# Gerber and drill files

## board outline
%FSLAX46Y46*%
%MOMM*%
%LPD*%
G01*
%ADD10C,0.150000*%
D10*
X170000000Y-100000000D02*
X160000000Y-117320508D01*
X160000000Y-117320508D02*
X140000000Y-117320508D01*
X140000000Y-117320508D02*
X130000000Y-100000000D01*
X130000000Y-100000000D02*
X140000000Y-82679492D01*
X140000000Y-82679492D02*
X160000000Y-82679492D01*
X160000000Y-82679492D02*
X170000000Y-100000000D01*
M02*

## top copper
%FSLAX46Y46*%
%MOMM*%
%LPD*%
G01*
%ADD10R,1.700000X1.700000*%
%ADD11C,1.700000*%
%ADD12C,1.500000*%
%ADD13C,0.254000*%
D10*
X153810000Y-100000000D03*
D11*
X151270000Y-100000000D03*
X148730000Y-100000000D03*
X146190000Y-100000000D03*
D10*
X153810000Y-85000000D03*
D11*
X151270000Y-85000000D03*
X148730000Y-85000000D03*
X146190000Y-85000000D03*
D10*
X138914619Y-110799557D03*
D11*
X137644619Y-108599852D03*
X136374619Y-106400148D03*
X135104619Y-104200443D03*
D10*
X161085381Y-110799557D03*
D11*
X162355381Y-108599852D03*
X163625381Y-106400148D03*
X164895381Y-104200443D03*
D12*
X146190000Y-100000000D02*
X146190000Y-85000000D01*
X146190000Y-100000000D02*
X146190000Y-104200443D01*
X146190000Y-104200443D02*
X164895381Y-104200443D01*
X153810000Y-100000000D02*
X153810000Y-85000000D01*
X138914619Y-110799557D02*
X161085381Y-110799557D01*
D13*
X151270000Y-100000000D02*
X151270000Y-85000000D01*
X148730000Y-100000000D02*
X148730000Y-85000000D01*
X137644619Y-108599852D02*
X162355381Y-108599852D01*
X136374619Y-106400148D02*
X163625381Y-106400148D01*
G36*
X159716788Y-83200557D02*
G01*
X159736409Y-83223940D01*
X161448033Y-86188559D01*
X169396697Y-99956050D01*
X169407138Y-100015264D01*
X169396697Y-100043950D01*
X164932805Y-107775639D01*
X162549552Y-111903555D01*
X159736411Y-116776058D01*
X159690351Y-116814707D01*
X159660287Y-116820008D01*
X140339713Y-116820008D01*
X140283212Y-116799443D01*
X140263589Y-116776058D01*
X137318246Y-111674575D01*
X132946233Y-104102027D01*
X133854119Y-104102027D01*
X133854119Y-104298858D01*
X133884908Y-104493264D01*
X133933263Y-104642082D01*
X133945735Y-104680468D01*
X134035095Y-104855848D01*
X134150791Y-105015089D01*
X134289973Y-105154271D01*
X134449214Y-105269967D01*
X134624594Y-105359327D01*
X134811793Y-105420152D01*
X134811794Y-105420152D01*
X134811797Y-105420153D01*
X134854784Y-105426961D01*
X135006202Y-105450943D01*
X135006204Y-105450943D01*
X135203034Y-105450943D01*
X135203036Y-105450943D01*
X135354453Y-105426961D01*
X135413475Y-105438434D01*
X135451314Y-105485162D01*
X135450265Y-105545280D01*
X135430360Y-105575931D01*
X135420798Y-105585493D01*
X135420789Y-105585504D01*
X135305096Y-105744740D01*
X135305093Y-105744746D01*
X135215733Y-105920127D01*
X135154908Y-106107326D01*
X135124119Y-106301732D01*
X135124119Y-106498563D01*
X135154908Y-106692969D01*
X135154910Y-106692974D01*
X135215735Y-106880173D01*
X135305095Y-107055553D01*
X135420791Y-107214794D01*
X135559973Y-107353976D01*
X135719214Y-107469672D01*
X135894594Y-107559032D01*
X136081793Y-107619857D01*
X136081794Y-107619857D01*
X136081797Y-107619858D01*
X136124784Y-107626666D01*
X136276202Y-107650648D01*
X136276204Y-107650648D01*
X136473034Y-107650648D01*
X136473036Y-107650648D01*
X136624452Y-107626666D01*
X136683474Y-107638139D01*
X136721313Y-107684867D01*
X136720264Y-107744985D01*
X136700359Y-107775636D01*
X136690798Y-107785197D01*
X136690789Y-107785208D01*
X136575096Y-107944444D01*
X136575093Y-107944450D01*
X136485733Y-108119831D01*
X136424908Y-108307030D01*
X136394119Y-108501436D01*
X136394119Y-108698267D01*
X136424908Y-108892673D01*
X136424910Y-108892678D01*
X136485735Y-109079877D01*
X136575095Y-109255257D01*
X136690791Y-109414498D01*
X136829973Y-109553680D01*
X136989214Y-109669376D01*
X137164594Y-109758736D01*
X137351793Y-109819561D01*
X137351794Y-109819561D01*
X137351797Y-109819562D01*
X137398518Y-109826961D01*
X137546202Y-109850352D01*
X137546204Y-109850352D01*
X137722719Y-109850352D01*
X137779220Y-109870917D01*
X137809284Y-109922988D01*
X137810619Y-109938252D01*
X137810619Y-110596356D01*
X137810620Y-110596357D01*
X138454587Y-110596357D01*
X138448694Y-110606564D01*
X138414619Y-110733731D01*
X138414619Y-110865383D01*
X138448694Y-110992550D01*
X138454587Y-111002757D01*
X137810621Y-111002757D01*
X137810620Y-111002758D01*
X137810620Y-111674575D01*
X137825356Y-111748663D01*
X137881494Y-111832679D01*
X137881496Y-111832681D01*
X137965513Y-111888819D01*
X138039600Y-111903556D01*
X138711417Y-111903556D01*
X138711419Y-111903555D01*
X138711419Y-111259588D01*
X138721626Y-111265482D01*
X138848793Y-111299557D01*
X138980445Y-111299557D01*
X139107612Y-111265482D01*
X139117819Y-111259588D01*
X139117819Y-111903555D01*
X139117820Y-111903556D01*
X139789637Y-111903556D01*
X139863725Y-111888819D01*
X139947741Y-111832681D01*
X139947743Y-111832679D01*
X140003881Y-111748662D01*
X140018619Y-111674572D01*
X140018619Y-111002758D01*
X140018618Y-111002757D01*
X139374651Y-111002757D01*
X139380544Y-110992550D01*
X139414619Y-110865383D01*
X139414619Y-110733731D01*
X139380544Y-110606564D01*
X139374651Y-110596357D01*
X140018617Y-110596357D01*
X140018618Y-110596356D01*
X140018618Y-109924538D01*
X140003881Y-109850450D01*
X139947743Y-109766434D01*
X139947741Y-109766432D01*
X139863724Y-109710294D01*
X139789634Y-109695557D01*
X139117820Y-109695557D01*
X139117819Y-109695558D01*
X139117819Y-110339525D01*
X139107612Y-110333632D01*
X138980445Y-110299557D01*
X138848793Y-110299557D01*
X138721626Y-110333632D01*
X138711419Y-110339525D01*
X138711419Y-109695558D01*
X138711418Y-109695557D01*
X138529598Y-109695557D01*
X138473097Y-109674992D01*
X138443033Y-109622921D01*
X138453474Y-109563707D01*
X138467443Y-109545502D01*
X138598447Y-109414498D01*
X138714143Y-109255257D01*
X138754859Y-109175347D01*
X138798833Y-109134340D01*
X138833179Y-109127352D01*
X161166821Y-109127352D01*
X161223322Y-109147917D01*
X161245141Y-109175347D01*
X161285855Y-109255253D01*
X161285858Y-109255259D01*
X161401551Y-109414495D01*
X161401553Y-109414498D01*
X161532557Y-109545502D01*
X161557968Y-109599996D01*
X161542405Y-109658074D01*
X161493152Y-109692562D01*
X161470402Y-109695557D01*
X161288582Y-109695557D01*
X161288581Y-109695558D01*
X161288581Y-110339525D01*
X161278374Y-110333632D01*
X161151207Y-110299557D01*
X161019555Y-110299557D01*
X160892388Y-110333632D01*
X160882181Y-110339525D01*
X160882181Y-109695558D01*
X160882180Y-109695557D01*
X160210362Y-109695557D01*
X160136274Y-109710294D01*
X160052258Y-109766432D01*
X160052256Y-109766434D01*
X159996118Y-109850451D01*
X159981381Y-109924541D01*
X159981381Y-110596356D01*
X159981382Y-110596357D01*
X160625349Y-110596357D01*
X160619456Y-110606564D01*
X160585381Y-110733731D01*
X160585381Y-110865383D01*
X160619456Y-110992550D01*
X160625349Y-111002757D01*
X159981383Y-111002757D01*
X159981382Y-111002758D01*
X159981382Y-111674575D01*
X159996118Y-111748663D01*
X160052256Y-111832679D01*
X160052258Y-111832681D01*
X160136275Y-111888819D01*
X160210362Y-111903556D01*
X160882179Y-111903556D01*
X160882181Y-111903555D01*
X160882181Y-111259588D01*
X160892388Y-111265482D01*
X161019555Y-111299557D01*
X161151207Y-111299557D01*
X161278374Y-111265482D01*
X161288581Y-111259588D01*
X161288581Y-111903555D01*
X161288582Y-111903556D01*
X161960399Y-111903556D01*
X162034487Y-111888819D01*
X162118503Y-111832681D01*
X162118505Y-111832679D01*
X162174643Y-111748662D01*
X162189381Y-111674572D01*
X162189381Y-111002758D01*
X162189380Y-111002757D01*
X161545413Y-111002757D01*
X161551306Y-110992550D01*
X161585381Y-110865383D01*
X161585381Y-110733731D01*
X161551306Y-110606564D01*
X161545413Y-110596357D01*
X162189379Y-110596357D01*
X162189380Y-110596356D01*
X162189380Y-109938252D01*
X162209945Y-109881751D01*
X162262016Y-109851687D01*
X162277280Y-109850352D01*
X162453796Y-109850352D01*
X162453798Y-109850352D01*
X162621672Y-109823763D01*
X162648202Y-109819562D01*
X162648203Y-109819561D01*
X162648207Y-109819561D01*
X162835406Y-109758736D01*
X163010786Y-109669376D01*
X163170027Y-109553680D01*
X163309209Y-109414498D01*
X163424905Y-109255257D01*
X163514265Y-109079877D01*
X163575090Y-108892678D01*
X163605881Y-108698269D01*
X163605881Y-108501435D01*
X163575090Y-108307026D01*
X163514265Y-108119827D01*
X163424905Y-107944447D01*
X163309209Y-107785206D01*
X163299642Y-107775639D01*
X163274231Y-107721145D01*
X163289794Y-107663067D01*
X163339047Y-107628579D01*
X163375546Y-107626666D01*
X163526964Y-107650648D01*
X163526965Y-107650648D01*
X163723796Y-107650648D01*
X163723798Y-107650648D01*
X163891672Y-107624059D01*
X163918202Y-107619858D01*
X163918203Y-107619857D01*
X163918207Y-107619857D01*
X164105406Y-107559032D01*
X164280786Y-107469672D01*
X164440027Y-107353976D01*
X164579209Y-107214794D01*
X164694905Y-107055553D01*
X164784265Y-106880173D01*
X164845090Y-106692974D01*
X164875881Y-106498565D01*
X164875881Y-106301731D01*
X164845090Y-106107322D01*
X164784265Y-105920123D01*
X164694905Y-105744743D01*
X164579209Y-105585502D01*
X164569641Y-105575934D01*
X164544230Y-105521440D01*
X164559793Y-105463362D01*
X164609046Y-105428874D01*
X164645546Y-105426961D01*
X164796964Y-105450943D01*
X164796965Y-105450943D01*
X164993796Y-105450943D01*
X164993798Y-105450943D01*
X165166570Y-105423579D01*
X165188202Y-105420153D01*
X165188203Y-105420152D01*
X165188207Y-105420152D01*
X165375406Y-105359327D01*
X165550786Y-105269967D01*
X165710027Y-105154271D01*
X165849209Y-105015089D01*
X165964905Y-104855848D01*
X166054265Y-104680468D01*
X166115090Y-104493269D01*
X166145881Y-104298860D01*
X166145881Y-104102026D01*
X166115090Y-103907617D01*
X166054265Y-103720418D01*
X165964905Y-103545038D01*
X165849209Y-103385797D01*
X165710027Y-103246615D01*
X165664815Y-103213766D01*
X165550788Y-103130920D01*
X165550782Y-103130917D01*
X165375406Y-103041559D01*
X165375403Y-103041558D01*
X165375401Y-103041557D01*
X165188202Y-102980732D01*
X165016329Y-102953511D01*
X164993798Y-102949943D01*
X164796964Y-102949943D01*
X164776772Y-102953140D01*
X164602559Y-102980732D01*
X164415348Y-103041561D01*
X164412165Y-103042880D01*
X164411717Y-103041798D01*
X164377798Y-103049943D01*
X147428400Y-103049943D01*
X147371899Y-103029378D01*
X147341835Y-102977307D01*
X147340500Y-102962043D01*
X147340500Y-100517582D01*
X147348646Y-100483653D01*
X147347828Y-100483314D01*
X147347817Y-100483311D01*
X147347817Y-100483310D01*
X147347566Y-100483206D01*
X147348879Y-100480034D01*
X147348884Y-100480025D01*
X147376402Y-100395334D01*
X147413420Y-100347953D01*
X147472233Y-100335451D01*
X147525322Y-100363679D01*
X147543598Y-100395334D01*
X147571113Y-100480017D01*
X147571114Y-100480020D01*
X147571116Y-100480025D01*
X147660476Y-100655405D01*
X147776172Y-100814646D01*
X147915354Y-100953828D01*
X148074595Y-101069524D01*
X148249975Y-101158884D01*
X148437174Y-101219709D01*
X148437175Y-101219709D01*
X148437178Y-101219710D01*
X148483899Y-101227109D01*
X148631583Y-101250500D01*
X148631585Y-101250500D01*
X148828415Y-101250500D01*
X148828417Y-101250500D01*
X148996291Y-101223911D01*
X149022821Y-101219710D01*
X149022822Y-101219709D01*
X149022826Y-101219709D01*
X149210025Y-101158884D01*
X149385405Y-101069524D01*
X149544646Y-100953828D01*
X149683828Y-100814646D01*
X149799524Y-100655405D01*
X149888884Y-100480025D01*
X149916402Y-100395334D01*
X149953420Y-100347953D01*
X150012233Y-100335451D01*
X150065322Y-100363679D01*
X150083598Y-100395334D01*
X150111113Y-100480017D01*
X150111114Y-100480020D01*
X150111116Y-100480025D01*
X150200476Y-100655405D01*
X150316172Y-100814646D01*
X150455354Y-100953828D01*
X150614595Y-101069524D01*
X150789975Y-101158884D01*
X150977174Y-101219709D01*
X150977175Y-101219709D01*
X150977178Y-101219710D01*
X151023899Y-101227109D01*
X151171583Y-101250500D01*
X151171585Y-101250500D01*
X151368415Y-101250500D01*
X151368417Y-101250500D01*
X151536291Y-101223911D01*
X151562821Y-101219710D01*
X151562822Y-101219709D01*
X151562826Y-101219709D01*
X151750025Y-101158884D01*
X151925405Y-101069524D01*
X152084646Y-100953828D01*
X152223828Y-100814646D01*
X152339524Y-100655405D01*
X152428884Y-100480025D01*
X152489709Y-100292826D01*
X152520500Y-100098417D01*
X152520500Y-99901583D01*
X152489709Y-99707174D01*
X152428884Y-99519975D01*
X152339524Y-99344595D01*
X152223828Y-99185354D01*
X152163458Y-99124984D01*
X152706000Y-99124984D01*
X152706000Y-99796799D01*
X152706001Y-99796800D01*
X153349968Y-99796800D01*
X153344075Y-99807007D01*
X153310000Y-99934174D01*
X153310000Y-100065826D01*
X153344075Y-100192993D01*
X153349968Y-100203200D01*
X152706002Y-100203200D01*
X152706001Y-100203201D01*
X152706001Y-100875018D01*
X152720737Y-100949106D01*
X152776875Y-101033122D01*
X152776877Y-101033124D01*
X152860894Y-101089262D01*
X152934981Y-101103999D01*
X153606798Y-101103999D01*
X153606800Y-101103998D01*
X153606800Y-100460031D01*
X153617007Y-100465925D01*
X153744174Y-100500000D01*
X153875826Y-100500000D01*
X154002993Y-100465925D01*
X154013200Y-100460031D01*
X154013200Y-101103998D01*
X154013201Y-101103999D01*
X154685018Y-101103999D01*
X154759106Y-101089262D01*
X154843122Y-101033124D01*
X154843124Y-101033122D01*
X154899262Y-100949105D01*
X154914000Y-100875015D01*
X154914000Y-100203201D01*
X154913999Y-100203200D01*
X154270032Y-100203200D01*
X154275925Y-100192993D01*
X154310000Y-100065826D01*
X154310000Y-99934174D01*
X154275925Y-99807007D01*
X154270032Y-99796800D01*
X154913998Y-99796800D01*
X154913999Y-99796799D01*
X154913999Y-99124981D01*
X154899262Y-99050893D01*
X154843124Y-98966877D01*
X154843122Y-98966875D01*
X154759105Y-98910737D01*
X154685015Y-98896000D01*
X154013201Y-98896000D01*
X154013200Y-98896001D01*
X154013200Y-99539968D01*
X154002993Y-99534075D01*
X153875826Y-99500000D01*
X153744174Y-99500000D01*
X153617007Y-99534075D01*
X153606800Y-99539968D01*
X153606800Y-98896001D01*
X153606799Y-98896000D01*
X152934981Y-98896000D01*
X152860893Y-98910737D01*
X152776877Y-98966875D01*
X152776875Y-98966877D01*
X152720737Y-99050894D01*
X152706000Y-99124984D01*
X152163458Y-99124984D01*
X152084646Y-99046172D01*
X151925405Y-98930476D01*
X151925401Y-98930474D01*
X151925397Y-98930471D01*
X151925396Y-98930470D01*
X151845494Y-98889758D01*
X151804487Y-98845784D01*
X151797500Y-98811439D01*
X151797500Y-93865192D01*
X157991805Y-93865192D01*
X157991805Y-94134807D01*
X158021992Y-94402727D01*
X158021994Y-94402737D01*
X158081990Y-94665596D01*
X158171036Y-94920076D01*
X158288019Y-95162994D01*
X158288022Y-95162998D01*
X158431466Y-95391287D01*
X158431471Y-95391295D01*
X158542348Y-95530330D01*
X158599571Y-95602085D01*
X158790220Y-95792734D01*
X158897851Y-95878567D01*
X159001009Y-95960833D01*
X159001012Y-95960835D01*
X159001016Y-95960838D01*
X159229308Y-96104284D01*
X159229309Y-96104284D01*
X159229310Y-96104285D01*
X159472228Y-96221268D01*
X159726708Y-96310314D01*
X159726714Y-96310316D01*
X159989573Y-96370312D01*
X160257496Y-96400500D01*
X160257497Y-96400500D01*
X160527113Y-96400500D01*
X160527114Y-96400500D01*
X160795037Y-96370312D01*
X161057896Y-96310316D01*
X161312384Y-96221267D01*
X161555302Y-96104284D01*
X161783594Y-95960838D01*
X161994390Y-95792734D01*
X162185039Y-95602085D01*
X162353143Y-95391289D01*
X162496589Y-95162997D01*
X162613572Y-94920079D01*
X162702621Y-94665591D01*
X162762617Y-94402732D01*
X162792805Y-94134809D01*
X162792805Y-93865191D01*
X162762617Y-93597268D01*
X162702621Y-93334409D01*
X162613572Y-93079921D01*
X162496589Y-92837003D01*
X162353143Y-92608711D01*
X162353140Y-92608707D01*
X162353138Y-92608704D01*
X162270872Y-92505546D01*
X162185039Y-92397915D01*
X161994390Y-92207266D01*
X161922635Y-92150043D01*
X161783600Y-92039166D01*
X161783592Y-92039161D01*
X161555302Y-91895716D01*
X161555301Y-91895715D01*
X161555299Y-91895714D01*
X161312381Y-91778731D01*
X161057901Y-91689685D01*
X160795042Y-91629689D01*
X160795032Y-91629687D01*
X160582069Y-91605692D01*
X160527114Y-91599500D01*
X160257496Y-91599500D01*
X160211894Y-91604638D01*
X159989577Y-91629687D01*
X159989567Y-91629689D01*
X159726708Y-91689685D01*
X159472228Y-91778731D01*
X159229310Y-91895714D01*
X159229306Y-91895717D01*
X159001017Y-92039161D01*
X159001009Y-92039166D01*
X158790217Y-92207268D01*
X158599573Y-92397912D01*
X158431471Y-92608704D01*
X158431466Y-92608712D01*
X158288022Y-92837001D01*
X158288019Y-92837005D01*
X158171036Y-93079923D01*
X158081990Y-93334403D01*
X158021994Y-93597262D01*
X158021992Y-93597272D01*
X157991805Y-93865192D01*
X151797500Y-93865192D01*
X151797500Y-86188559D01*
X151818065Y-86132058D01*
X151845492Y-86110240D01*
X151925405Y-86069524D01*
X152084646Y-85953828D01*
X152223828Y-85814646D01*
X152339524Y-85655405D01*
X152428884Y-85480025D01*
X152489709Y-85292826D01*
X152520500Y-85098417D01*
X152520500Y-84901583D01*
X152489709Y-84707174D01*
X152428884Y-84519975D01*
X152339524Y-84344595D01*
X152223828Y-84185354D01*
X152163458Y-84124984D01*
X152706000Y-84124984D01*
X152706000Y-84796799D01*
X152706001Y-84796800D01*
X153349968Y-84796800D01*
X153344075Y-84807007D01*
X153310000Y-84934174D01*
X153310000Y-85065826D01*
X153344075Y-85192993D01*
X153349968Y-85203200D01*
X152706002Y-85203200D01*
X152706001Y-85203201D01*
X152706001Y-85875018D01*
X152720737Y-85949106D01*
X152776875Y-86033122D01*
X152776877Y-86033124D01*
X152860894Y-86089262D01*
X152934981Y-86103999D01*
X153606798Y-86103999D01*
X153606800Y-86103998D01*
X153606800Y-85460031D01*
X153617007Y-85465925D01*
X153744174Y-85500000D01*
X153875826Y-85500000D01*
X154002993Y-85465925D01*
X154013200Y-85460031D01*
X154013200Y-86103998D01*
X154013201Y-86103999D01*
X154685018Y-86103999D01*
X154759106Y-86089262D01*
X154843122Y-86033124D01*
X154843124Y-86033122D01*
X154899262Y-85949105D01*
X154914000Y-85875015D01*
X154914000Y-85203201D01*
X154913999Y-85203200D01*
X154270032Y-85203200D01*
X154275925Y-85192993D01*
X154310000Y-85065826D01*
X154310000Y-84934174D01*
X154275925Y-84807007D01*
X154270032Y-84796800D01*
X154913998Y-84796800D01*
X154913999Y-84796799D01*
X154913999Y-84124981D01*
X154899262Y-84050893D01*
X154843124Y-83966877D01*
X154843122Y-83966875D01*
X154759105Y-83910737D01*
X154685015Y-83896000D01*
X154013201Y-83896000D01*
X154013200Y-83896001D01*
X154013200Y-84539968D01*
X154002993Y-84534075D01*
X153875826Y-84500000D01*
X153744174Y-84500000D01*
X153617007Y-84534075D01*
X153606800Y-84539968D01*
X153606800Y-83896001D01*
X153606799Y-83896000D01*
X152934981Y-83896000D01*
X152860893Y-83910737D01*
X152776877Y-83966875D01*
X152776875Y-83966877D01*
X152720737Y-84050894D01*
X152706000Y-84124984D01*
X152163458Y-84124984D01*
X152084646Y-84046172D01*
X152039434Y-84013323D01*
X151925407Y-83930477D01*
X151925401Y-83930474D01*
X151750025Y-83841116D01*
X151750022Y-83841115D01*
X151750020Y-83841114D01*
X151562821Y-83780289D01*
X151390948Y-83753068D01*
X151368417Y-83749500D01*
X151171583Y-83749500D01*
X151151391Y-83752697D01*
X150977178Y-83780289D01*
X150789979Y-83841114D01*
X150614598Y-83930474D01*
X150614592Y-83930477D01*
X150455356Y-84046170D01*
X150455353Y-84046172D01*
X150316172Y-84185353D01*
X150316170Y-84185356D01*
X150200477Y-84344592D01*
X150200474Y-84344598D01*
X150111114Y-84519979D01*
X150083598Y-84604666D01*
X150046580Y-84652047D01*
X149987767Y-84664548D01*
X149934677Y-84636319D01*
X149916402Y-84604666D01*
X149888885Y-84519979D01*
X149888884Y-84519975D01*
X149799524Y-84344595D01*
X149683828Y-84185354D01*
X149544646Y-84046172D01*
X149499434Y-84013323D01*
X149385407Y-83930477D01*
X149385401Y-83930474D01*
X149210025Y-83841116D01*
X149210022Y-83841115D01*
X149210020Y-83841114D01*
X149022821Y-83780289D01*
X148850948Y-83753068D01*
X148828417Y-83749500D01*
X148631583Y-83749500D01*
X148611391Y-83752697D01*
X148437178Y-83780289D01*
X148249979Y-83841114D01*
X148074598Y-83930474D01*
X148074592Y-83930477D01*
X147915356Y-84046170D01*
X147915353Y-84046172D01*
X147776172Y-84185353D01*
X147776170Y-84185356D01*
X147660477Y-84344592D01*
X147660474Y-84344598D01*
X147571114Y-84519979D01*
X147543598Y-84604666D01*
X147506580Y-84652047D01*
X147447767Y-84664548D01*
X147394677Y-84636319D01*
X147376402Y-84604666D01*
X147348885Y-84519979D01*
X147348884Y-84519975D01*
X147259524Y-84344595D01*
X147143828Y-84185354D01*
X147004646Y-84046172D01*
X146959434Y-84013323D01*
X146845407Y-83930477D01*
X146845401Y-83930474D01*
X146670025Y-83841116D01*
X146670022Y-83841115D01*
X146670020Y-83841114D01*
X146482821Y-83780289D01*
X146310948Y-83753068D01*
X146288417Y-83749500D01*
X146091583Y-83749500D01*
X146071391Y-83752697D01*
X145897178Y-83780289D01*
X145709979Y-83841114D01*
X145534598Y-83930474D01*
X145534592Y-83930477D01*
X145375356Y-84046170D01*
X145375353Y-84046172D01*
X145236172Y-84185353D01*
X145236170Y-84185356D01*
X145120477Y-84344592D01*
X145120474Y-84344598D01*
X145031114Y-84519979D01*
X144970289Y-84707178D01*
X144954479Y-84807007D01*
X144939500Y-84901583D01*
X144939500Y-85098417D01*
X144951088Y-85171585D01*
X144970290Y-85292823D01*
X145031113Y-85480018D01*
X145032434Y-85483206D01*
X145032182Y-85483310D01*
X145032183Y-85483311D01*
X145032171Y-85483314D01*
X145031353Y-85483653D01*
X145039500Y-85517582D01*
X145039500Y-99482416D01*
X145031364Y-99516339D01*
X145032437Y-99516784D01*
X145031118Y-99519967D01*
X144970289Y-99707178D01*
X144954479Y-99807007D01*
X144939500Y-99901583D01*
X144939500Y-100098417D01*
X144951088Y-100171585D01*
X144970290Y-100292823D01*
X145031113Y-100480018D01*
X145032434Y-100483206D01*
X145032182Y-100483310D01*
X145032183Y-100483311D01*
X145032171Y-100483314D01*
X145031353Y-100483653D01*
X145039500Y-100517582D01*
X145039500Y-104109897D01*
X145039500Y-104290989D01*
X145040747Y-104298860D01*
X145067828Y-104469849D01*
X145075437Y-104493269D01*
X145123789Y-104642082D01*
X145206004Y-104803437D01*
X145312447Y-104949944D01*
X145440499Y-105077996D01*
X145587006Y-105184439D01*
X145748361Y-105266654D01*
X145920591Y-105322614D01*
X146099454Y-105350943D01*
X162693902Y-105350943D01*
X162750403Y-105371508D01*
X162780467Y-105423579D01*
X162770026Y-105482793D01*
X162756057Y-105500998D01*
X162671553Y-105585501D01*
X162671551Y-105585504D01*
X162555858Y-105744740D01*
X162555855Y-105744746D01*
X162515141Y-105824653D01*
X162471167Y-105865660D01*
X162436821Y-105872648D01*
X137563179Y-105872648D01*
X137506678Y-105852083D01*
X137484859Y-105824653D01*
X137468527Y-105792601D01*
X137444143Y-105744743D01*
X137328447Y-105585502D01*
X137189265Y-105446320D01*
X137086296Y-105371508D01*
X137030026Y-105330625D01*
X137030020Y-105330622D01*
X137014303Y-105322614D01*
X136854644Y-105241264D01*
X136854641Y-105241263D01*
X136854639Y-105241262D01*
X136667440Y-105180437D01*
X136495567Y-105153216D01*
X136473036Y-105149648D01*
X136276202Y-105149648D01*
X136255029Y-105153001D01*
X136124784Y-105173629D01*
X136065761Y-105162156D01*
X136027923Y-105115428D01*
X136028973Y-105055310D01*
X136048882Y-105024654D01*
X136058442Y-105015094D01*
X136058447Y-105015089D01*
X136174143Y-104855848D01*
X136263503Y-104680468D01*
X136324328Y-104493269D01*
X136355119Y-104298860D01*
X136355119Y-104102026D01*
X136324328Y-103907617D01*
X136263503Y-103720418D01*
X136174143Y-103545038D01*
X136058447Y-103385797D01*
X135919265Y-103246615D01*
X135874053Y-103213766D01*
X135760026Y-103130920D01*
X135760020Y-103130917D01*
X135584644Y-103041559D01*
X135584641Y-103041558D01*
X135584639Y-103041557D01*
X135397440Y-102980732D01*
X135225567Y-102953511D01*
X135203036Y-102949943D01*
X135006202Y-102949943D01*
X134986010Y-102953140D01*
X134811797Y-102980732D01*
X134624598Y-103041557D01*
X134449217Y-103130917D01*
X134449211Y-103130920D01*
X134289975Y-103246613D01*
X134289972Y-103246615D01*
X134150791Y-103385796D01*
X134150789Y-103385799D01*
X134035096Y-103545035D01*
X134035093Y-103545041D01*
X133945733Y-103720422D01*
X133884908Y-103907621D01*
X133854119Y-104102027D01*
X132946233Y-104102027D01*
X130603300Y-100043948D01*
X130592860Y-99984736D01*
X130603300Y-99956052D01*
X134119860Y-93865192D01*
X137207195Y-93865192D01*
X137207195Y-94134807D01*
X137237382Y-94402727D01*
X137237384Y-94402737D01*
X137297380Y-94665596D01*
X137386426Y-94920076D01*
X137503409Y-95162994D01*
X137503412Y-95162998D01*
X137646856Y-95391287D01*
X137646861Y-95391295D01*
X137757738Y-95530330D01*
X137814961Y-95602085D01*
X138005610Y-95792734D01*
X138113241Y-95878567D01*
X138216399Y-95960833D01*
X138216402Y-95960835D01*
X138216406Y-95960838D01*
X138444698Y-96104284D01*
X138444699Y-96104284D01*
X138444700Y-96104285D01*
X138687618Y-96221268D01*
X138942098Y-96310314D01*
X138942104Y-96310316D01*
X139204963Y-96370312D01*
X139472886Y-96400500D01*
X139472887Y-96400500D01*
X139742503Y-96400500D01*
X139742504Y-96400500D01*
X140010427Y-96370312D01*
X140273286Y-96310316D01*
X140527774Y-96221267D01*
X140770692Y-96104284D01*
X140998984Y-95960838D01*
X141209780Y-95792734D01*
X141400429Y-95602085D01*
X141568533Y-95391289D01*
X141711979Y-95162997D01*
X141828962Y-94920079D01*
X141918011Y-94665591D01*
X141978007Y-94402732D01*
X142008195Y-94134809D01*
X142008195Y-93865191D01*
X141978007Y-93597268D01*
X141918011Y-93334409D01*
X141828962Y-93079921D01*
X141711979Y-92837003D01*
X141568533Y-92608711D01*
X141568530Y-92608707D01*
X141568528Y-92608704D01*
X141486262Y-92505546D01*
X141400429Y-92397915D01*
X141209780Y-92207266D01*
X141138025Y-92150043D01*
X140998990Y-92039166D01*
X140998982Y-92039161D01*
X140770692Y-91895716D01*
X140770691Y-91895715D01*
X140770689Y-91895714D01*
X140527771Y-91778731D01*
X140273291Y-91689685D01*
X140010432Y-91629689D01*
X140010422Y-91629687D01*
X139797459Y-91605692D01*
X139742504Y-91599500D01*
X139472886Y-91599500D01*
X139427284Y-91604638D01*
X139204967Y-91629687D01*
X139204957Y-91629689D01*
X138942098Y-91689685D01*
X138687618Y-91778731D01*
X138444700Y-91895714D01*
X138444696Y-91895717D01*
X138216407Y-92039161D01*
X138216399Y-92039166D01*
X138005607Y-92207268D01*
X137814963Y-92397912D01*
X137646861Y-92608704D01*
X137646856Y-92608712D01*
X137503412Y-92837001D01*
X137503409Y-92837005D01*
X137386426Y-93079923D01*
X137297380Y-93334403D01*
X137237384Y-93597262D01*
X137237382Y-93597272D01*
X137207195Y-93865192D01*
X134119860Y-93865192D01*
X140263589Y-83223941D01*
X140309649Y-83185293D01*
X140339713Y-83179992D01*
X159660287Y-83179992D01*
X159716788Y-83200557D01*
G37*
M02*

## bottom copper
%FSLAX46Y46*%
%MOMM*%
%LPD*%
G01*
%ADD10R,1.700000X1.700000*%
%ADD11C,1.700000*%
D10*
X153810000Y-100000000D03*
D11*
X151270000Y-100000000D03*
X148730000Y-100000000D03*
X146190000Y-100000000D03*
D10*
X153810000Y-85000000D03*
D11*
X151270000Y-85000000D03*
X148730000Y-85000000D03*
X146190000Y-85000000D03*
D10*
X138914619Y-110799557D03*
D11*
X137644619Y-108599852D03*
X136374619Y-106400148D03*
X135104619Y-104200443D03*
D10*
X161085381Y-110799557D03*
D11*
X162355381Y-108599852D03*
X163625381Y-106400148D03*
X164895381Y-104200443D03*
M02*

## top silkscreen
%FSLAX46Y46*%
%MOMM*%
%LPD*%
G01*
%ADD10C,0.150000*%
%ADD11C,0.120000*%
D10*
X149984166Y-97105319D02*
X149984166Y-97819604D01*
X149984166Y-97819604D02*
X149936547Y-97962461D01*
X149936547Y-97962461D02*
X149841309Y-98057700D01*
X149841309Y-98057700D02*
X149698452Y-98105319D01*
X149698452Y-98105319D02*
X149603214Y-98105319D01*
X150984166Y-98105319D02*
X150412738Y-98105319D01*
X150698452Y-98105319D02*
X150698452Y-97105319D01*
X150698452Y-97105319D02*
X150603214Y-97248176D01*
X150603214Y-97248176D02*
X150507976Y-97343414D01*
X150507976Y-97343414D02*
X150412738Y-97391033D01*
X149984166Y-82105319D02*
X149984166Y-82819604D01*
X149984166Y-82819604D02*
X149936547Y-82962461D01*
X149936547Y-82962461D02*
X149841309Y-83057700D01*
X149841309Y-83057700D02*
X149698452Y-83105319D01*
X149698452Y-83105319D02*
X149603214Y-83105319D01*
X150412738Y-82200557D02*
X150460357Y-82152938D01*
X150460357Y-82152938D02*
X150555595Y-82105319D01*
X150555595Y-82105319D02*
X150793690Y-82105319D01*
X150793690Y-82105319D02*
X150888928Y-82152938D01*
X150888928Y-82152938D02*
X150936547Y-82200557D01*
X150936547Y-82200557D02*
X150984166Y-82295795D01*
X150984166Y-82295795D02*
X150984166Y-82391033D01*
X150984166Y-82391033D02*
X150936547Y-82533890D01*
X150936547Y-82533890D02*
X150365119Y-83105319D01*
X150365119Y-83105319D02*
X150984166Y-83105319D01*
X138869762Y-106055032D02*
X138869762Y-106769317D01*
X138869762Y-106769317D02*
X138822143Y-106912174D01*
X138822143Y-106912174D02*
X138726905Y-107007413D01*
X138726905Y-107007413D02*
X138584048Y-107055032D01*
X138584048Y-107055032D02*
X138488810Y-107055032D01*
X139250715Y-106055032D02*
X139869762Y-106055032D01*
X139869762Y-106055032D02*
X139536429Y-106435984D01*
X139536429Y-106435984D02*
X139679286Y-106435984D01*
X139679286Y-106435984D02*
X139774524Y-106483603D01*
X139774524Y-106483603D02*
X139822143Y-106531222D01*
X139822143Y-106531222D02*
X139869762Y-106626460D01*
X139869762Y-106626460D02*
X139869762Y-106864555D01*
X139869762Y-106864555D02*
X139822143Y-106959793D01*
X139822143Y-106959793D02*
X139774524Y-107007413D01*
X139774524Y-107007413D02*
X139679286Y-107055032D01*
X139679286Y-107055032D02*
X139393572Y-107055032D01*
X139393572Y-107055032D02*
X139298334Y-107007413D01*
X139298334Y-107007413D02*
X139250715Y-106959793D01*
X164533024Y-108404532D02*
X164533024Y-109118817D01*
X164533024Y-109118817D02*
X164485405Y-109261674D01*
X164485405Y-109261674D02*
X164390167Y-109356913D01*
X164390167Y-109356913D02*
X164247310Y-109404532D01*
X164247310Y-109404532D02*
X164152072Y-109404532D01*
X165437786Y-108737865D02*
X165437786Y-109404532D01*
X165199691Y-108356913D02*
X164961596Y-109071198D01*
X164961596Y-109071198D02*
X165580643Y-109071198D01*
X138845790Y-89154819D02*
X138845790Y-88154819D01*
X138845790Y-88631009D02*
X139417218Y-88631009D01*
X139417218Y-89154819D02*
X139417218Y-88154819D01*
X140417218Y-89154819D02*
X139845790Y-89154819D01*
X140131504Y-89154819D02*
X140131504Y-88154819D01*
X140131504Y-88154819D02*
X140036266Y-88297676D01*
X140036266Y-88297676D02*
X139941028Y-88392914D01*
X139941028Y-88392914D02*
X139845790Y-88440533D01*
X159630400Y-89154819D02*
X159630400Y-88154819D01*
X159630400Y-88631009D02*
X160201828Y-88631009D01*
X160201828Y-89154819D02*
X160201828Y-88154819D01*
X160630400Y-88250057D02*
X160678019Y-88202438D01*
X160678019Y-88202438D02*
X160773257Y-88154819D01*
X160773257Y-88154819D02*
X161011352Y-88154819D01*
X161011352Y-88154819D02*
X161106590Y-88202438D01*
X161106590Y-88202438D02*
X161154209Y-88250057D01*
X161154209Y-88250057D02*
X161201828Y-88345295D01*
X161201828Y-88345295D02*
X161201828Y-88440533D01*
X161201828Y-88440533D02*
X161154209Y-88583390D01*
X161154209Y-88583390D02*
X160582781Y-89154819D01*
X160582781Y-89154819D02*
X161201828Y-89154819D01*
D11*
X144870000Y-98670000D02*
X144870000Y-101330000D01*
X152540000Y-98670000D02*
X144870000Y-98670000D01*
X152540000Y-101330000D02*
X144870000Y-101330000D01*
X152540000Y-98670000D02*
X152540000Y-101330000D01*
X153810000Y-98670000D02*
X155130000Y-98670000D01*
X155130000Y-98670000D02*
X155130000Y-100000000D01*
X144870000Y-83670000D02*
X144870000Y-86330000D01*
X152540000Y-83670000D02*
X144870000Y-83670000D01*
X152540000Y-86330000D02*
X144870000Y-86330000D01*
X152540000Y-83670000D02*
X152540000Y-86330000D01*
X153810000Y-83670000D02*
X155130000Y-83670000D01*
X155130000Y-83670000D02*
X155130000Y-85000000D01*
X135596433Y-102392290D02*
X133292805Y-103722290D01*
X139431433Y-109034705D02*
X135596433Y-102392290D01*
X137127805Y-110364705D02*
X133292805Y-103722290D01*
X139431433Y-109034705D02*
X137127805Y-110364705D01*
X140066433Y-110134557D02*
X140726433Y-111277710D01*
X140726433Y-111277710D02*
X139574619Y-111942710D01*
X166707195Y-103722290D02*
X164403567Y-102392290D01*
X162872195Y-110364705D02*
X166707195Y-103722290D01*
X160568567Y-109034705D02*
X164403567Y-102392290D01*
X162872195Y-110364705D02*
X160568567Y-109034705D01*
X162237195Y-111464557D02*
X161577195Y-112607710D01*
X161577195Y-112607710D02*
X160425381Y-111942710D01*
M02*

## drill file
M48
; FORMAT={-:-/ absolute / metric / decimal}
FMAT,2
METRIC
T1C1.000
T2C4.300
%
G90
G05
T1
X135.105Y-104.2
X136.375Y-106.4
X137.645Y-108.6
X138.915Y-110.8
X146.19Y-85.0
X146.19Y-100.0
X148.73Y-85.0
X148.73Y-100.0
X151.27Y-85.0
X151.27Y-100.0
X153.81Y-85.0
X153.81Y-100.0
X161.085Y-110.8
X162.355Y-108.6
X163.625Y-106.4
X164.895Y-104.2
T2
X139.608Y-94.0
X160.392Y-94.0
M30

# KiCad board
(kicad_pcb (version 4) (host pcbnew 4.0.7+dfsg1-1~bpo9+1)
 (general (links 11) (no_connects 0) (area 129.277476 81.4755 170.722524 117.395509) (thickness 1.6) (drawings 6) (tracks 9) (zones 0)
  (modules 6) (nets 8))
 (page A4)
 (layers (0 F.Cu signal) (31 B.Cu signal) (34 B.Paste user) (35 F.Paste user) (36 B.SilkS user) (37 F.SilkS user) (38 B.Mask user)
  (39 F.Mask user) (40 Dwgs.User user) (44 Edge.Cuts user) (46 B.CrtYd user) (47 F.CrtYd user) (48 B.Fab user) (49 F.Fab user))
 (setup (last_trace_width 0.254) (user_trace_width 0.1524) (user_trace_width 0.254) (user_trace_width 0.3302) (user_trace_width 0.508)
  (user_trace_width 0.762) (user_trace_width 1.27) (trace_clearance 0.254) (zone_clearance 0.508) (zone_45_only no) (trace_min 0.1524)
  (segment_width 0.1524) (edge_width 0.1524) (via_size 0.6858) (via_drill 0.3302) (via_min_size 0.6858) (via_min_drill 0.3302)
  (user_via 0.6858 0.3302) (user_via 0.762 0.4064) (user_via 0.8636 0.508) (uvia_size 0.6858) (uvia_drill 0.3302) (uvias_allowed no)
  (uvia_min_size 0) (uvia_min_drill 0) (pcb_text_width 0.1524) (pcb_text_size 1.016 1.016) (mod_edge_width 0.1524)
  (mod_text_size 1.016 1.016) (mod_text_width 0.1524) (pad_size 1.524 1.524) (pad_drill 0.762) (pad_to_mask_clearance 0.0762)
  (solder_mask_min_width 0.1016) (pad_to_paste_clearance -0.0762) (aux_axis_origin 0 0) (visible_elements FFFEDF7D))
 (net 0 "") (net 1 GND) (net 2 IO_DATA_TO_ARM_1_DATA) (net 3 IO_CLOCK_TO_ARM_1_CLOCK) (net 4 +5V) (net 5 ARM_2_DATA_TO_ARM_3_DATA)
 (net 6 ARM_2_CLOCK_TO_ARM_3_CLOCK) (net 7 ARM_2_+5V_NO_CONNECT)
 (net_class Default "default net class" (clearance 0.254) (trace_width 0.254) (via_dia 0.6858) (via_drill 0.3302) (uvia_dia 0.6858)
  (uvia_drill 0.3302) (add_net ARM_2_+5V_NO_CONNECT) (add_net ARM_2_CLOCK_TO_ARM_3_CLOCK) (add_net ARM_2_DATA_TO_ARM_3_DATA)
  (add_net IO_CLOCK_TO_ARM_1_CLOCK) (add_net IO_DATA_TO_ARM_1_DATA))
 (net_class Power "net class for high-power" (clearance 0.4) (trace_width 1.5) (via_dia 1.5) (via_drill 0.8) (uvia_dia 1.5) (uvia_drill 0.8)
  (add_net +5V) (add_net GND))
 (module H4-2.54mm (layer F.Cu) (at 150 100 270)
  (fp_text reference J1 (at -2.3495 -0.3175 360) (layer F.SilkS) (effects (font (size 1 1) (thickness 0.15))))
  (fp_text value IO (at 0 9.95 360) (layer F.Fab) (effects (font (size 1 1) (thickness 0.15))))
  (fp_line (start -1.33 5.13) (end 1.33 5.13) (layer F.SilkS) (width 0.12))
  (fp_line (start -1.33 -2.54) (end -1.33 5.13) (layer F.SilkS) (width 0.12))
  (fp_line (start 1.33 -2.54) (end 1.33 5.13) (layer F.SilkS) (width 0.12))
  (fp_line (start -1.33 -2.54) (end 1.33 -2.54) (layer F.SilkS) (width 0.12))
  (fp_line (start -1.33 -3.81) (end -1.33 -5.13) (layer F.SilkS) (width 0.12))
  (fp_line (start -1.33 -5.13) (end 0 -5.13) (layer F.SilkS) (width 0.12))
  (pad 1 thru_hole rect (at 0 -3.81) (size 1.7 1.7) (drill 1) (layers *.Cu *.Paste *.Mask) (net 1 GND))
  (pad 2 thru_hole circle (at 0 -1.27) (size 1.7 1.7) (drill 1) (layers *.Cu *.Paste *.Mask) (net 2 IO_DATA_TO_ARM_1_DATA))
  (pad 3 thru_hole circle (at 0 1.27) (size 1.7 1.7) (drill 1) (layers *.Cu *.Paste *.Mask) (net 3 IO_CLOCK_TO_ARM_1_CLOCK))
  (pad 4 thru_hole circle (at 0 3.81) (size 1.7 1.7) (drill 1) (layers *.Cu *.Paste *.Mask) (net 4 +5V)))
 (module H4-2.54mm (layer F.Cu) (at 150 85 270)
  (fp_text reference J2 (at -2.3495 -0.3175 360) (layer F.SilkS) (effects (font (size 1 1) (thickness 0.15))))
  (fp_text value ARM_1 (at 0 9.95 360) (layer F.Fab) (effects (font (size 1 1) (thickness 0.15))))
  (fp_line (start -1.33 5.13) (end 1.33 5.13) (layer F.SilkS) (width 0.12))
  (fp_line (start -1.33 -2.54) (end -1.33 5.13) (layer F.SilkS) (width 0.12))
  (fp_line (start 1.33 -2.54) (end 1.33 5.13) (layer F.SilkS) (width 0.12))
  (fp_line (start -1.33 -2.54) (end 1.33 -2.54) (layer F.SilkS) (width 0.12))
  (fp_line (start -1.33 -3.81) (end -1.33 -5.13) (layer F.SilkS) (width 0.12))
  (fp_line (start -1.33 -5.13) (end 0 -5.13) (layer F.SilkS) (width 0.12))
  (pad 1 thru_hole rect (at 0 -3.81) (size 1.7 1.7) (drill 1) (layers *.Cu *.Paste *.Mask) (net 1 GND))
  (pad 2 thru_hole circle (at 0 -1.27) (size 1.7 1.7) (drill 1) (layers *.Cu *.Paste *.Mask) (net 2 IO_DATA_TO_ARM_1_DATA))
  (pad 3 thru_hole circle (at 0 1.27) (size 1.7 1.7) (drill 1) (layers *.Cu *.Paste *.Mask) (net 3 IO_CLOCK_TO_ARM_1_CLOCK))
  (pad 4 thru_hole circle (at 0 3.81) (size 1.7 1.7) (drill 1) (layers *.Cu *.Paste *.Mask) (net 4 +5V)))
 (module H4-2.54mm (layer F.Cu) (at 137.009619 107.5 210)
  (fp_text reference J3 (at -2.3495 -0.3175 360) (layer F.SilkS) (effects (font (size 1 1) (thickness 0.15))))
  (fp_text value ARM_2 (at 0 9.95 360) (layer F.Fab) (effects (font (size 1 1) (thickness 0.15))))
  (fp_line (start -1.33 5.13) (end 1.33 5.13) (layer F.SilkS) (width 0.12))
  (fp_line (start -1.33 -2.54) (end -1.33 5.13) (layer F.SilkS) (width 0.12))
  (fp_line (start 1.33 -2.54) (end 1.33 5.13) (layer F.SilkS) (width 0.12))
  (fp_line (start -1.33 -2.54) (end 1.33 -2.54) (layer F.SilkS) (width 0.12))
  (fp_line (start -1.33 -3.81) (end -1.33 -5.13) (layer F.SilkS) (width 0.12))
  (fp_line (start -1.33 -5.13) (end 0 -5.13) (layer F.SilkS) (width 0.12))
  (pad 1 thru_hole rect (at 0 -3.81) (size 1.7 1.7) (drill 1) (layers *.Cu *.Paste *.Mask) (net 1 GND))
  (pad 2 thru_hole circle (at 0 -1.27) (size 1.7 1.7) (drill 1) (layers *.Cu *.Paste *.Mask) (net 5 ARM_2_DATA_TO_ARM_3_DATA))
  (pad 3 thru_hole circle (at 0 1.27) (size 1.7 1.7) (drill 1) (layers *.Cu *.Paste *.Mask) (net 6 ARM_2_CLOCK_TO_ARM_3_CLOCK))
  (pad 4 thru_hole circle (at 0 3.81) (size 1.7 1.7) (drill 1) (layers *.Cu *.Paste *.Mask) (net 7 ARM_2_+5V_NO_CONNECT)))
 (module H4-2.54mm (layer F.Cu) (at 162.990381 107.5 150)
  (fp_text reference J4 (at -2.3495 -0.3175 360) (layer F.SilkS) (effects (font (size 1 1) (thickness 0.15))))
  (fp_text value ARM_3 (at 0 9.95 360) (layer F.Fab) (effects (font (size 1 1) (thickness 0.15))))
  (fp_line (start -1.33 5.13) (end 1.33 5.13) (layer F.SilkS) (width 0.12))
  (fp_line (start -1.33 -2.54) (end -1.33 5.13) (layer F.SilkS) (width 0.12))
  (fp_line (start 1.33 -2.54) (end 1.33 5.13) (layer F.SilkS) (width 0.12))
  (fp_line (start -1.33 -2.54) (end 1.33 -2.54) (layer F.SilkS) (width 0.12))
  (fp_line (start -1.33 -3.81) (end -1.33 -5.13) (layer F.SilkS) (width 0.12))
  (fp_line (start -1.33 -5.13) (end 0 -5.13) (layer F.SilkS) (width 0.12))
  (pad 1 thru_hole rect (at 0 -3.81) (size 1.7 1.7) (drill 1) (layers *.Cu *.Paste *.Mask) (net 1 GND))
  (pad 2 thru_hole circle (at 0 -1.27) (size 1.7 1.7) (drill 1) (layers *.Cu *.Paste *.Mask) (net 5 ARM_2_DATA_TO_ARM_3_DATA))
  (pad 3 thru_hole circle (at 0 1.27) (size 1.7 1.7) (drill 1) (layers *.Cu *.Paste *.Mask) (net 6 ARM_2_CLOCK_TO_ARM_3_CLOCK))
  (pad 4 thru_hole circle (at 0 3.81) (size 1.7 1.7) (drill 1) (layers *.Cu *.Paste *.Mask) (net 4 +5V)))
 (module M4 (layer F.Cu) (at 139.607695 94)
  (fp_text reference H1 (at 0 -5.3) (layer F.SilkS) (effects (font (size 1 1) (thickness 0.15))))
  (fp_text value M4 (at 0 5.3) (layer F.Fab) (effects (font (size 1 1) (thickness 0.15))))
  (pad 1 np_thru_hole circle (at 0 0) (size 4.3 4.3) (drill 4.3) (layers *.Cu *.Mask) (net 1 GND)))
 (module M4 (layer F.Cu) (at 160.392305 94)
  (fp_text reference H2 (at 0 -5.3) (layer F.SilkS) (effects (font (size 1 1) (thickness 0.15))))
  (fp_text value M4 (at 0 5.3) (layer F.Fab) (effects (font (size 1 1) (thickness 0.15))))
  (pad 1 np_thru_hole circle (at 0 0) (size 4.3 4.3) (drill 4.3) (layers *.Cu *.Mask) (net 1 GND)))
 (gr_line (start 170 100) (end 160 117.320508) (angle 90) (layer Edge.Cuts) (width 0.15))
 (gr_line (start 160 117.320508) (end 140 117.320508) (angle 90) (layer Edge.Cuts) (width 0.15))
 (gr_line (start 140 117.320508) (end 130 100) (angle 90) (layer Edge.Cuts) (width 0.15))
 (gr_line (start 130 100) (end 140 82.679492) (angle 90) (layer Edge.Cuts) (width 0.15))
 (gr_line (start 140 82.679492) (end 160 82.679492) (angle 90) (layer Edge.Cuts) (width 0.15))
 (gr_line (start 160 82.679492) (end 170 100) (angle 90) (layer Edge.Cuts) (width 0.15))
 (segment (start 146.19 100) (end 146.19 85) (width 1.5) (layer F.Cu) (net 4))
 (segment (start 146.19 100) (end 146.19 104.200443) (width 1.5) (layer F.Cu) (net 4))
 (segment (start 146.19 104.200443) (end 164.895381 104.200443) (width 1.5) (layer F.Cu) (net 4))
 (segment (start 153.81 100) (end 153.81 85) (width 1.5) (layer F.Cu) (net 1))
 (segment (start 138.914619 110.799557) (end 161.085381 110.799557) (width 1.5) (layer F.Cu) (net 1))
 (segment (start 151.27 100) (end 151.27 85) (width 0.254) (layer F.Cu) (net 2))
 (segment (start 148.73 100) (end 148.73 85) (width 0.254) (layer F.Cu) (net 3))
 (segment (start 137.644619 108.599852) (end 162.355381 108.599852) (width 0.254) (layer F.Cu) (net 5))
 (segment (start 136.374619 106.400148) (end 163.625381 106.400148) (width 0.254) (layer F.Cu) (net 6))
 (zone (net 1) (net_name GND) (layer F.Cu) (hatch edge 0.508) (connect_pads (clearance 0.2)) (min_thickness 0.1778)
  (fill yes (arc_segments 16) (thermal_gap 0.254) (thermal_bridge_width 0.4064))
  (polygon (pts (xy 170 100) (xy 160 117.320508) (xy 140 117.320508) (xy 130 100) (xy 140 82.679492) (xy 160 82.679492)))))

